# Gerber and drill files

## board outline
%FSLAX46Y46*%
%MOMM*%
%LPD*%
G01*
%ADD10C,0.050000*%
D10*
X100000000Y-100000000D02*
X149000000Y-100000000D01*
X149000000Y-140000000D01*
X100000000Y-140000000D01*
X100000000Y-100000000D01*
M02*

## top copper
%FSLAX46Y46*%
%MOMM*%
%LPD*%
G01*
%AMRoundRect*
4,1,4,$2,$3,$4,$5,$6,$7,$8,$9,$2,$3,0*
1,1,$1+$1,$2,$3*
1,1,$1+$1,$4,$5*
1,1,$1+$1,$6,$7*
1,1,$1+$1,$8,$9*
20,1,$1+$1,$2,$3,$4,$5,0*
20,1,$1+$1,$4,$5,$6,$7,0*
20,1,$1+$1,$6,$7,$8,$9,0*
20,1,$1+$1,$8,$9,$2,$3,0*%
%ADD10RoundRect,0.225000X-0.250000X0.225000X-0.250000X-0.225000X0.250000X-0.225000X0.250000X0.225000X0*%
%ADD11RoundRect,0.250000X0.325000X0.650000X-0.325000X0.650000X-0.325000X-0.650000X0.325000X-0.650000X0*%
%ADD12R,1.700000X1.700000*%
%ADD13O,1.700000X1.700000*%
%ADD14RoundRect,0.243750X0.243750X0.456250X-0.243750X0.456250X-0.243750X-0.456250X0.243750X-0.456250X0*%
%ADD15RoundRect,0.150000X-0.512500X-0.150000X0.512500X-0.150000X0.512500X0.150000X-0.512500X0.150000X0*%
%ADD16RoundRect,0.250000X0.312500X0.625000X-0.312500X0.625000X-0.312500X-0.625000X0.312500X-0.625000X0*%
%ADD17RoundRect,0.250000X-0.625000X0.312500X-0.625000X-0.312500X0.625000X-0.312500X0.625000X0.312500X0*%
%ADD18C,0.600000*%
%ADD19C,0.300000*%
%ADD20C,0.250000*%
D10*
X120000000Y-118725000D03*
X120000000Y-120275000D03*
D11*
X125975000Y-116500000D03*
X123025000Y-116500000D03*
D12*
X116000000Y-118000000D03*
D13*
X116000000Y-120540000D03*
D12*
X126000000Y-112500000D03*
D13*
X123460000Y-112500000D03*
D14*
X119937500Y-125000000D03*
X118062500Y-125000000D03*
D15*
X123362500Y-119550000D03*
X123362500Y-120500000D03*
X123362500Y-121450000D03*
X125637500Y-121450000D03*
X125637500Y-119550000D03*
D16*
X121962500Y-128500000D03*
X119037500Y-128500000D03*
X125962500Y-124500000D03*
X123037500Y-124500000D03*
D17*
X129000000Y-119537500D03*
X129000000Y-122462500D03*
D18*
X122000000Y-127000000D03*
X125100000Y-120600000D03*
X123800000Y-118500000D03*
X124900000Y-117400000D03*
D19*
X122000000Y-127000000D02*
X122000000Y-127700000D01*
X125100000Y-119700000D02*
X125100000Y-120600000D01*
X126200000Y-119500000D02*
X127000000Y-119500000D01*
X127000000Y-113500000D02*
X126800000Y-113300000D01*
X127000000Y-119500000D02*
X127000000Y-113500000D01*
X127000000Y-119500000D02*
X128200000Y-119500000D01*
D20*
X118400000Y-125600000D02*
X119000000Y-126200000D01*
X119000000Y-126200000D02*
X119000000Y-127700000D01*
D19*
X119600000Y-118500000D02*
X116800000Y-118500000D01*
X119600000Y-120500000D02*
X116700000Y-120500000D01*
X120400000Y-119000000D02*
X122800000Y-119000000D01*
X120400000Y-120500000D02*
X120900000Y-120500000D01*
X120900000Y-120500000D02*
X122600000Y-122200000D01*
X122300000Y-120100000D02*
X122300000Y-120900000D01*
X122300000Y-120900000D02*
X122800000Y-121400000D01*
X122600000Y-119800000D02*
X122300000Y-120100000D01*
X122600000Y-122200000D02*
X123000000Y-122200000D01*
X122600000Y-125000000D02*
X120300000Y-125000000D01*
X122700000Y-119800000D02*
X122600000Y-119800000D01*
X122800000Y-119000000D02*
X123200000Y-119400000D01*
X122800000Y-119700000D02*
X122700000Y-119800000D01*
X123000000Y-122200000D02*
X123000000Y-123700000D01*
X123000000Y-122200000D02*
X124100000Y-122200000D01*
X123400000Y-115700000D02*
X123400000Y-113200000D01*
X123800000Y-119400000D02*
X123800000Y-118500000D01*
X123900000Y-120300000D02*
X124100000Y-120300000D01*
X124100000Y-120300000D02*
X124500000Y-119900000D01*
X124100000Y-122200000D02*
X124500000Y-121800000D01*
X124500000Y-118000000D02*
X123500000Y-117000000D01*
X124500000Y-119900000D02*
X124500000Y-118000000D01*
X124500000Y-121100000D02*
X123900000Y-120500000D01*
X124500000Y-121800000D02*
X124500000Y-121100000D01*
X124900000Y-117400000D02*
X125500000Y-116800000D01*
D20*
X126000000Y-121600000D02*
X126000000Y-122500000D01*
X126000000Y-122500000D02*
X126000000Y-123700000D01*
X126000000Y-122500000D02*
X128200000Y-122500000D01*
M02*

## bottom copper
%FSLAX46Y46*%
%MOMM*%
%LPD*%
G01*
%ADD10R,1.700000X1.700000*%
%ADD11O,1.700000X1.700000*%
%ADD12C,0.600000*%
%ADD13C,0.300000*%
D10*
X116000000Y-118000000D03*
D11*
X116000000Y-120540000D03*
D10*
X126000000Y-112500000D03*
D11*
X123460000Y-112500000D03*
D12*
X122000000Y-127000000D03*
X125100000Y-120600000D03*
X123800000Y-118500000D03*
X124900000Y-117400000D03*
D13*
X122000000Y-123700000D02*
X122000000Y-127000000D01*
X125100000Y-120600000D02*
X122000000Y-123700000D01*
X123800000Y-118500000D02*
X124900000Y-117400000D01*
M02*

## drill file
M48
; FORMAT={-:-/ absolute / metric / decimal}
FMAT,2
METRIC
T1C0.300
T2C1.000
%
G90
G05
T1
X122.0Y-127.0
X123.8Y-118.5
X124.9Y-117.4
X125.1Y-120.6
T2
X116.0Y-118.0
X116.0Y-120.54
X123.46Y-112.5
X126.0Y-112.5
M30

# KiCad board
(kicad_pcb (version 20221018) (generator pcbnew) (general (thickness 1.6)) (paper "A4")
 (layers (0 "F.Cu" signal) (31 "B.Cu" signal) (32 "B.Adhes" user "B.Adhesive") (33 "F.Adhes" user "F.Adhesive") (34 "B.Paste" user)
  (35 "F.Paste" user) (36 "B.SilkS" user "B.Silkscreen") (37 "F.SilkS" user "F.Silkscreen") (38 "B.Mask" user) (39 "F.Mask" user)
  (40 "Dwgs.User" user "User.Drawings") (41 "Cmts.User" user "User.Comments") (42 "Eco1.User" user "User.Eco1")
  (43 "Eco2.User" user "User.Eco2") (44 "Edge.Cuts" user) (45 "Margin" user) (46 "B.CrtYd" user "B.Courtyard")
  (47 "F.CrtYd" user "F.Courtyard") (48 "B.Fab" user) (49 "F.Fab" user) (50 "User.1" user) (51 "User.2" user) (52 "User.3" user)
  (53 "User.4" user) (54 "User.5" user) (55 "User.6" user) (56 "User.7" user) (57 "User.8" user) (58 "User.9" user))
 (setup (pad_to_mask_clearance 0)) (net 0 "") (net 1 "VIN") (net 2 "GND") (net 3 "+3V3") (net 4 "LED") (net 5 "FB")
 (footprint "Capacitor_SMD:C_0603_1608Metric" (layer "F.Cu") (at 120 119.5 -90)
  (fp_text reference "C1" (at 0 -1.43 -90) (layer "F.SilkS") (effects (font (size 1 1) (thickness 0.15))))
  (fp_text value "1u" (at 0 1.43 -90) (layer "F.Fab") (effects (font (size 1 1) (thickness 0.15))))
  (pad "1" smd roundrect (at -0.775 0 270) (size 0.9 0.95) (layers "F.Cu" "F.Paste" "F.Mask") (roundrect_rratio 0.25) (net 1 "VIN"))
  (pad "2" smd roundrect (at 0.775 0 270) (size 0.9 0.95) (layers "F.Cu" "F.Paste" "F.Mask") (roundrect_rratio 0.25) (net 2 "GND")))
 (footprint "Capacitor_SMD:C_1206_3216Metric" (layer "F.Cu") (at 124.5 116.5 180)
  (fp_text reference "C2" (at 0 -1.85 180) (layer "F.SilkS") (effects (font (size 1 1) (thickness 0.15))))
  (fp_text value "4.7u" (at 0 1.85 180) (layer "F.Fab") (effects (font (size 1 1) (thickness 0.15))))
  (pad "1" smd roundrect (at -1.475 0 180) (size 1.15 1.8) (layers "F.Cu" "F.Paste" "F.Mask") (roundrect_rratio 0.217391) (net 1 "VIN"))
  (pad "2" smd roundrect (at 1.475 0 180) (size 1.15 1.8) (layers "F.Cu" "F.Paste" "F.Mask") (roundrect_rratio 0.217391) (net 2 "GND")))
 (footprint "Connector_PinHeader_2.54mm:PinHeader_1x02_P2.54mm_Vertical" (layer "F.Cu") (at 116 118)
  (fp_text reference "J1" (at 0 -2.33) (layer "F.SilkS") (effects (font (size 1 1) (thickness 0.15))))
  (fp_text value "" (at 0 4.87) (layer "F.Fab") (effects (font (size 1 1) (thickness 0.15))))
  (pad "1" thru_hole rect (at 0 0) (size 1.7 1.7) (drill 1) (layers "*.Cu" "*.Mask") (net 1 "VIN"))
  (pad "2" thru_hole oval (at 0 2.54) (size 1.7 1.7) (drill 1) (layers "*.Cu" "*.Mask") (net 2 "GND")))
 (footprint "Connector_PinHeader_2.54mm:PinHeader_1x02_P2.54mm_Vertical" (layer "F.Cu") (at 126 112.5 -90)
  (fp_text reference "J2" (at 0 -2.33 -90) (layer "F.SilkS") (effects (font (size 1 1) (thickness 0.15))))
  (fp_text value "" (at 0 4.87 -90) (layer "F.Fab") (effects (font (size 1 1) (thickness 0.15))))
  (pad "1" thru_hole rect (at 0 0 270) (size 1.7 1.7) (drill 1) (layers "*.Cu" "*.Mask") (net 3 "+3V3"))
  (pad "2" thru_hole oval (at 0 2.54 270) (size 1.7 1.7) (drill 1) (layers "*.Cu" "*.Mask") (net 2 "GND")))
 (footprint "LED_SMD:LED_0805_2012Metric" (layer "F.Cu") (at 119 125 180)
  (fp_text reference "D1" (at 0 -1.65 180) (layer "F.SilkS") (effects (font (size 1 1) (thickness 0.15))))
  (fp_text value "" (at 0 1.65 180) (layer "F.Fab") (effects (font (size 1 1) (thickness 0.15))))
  (pad "1" smd roundrect (at -0.9375 0 180) (size 0.975 1.4) (layers "F.Cu" "F.Paste" "F.Mask") (roundrect_rratio 0.25) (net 2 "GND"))
  (pad "2" smd roundrect (at 0.9375 0 180) (size 0.975 1.4) (layers "F.Cu" "F.Paste" "F.Mask") (roundrect_rratio 0.25) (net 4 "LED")))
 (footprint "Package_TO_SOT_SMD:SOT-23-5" (layer "F.Cu") (at 124.5 120.5)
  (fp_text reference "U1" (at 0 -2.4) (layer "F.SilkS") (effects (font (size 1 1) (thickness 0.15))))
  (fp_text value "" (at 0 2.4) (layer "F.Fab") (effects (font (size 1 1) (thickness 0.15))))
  (pad "1" smd roundrect (at -1.1375 -0.95) (size 1.325 0.6) (layers "F.Cu" "F.Paste" "F.Mask") (roundrect_rratio 0.25) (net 1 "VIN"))
  (pad "2" smd roundrect (at -1.1375 0) (size 1.325 0.6) (layers "F.Cu" "F.Paste" "F.Mask") (roundrect_rratio 0.25) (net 2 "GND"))
  (pad "3" smd roundrect (at -1.1375 0.95) (size 1.325 0.6) (layers "F.Cu" "F.Paste" "F.Mask") (roundrect_rratio 0.25) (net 1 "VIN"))
  (pad "4" smd roundrect (at 1.1375 0.95) (size 1.325 0.6) (layers "F.Cu" "F.Paste" "F.Mask") (roundrect_rratio 0.25) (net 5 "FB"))
  (pad "5" smd roundrect (at 1.1375 -0.95) (size 1.325 0.6) (layers "F.Cu" "F.Paste" "F.Mask") (roundrect_rratio 0.25) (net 3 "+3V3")))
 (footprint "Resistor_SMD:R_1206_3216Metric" (layer "F.Cu") (at 120.5 128.5 180)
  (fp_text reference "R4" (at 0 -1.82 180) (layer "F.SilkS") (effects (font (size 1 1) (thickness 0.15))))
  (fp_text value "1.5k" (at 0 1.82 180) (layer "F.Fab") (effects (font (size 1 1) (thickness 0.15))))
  (pad "1" smd roundrect (at -1.4625 0 180) (size 1.125 1.75) (layers "F.Cu" "F.Paste" "F.Mask") (roundrect_rratio 0.222222) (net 3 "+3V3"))
  (pad "2" smd roundrect (at 1.4625 0 180) (size 1.125 1.75) (layers "F.Cu" "F.Paste" "F.Mask") (roundrect_rratio 0.222222) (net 4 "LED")))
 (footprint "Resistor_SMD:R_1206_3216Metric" (layer "F.Cu") (at 124.5 124.5 180)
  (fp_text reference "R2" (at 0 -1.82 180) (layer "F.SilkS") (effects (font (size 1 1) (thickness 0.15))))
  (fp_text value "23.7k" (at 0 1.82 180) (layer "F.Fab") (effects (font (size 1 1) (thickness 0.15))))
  (pad "1" smd roundrect (at -1.4625 0 180) (size 1.125 1.75) (layers "F.Cu" "F.Paste" "F.Mask") (roundrect_rratio 0.222222) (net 5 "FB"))
  (pad "2" smd roundrect (at 1.4625 0 180) (size 1.125 1.75) (layers "F.Cu" "F.Paste" "F.Mask") (roundrect_rratio 0.222222) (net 2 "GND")))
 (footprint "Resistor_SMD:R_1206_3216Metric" (layer "F.Cu") (at 129 121 -90)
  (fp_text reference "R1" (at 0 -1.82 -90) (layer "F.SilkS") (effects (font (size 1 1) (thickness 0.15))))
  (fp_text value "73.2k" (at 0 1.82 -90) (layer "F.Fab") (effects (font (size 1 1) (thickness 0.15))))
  (pad "1" smd roundrect (at -1.4625 0 270) (size 1.125 1.75) (layers "F.Cu" "F.Paste" "F.Mask") (roundrect_rratio 0.222222) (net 3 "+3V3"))
  (pad "2" smd roundrect (at 1.4625 0 270) (size 1.125 1.75) (layers "F.Cu" "F.Paste" "F.Mask") (roundrect_rratio 0.222222) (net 5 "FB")))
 (gr_rect (start 100 100) (end 149 140) (stroke (width 0.05) (type default)) (fill none) (layer "Edge.Cuts"))
 (segment (start 122 127) (end 122 127.7) (width 0.3) (layer "F.Cu") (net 3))
 (segment (start 125.1 119.7) (end 125.1 120.6) (width 0.3) (layer "F.Cu") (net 3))
 (segment (start 126.2 119.5) (end 127 119.5) (width 0.3) (layer "F.Cu") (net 3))
 (segment (start 127 113.5) (end 126.8 113.3) (width 0.3) (layer "F.Cu") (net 3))
 (segment (start 127 119.5) (end 127 113.5) (width 0.3) (layer "F.Cu") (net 3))
 (segment (start 127 119.5) (end 128.2 119.5) (width 0.3) (layer "F.Cu") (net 3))
 (via (at 122 127) (size 0.6) (drill 0.3) (layers "F.Cu" "B.Cu") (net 3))
 (via (at 125.1 120.6) (size 0.6) (drill 0.3) (layers "F.Cu" "B.Cu") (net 3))
 (segment (start 118.4 125.6) (end 119 126.2) (width 0.25) (layer "F.Cu") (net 4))
 (segment (start 119 126.2) (end 119 127.7) (width 0.25) (layer "F.Cu") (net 4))
 (segment (start 119.6 118.5) (end 116.8 118.5) (width 0.3) (layer "F.Cu") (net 1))
 (segment (start 119.6 120.5) (end 116.7 120.5) (width 0.3) (layer "F.Cu") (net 2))
 (segment (start 120.4 119) (end 122.8 119) (width 0.3) (layer "F.Cu") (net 1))
 (segment (start 120.4 120.5) (end 120.9 120.5) (width 0.3) (layer "F.Cu") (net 2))
 (segment (start 120.9 120.5) (end 122.6 122.2) (width 0.3) (layer "F.Cu") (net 2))
 (segment (start 122 123.7) (end 122 127) (width 0.3) (layer "B.Cu") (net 3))
 (segment (start 122.3 120.1) (end 122.3 120.9) (width 0.3) (layer "F.Cu") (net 1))
 (segment (start 122.3 120.9) (end 122.8 121.4) (width 0.3) (layer "F.Cu") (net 1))
 (segment (start 122.6 119.8) (end 122.3 120.1) (width 0.3) (layer "F.Cu") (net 1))
 (segment (start 122.6 122.2) (end 123 122.2) (width 0.3) (layer "F.Cu") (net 2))
 (segment (start 122.6 125) (end 120.3 125) (width 0.3) (layer "F.Cu") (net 2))
 (segment (start 122.7 119.8) (end 122.6 119.8) (width 0.3) (layer "F.Cu") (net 1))
 (segment (start 122.8 119) (end 123.2 119.4) (width 0.3) (layer "F.Cu") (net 1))
 (segment (start 122.8 119.7) (end 122.7 119.8) (width 0.3) (layer "F.Cu") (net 1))
 (segment (start 123 122.2) (end 123 123.7) (width 0.3) (layer "F.Cu") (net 2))
 (segment (start 123 122.2) (end 124.1 122.2) (width 0.3) (layer "F.Cu") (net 2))
 (segment (start 123.4 115.7) (end 123.4 113.2) (width 0.3) (layer "F.Cu") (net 2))
 (segment (start 123.8 119.4) (end 123.8 118.5) (width 0.3) (layer "F.Cu") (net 1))
 (segment (start 123.9 120.3) (end 124.1 120.3) (width 0.3) (layer "F.Cu") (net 2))
 (segment (start 124.1 120.3) (end 124.5 119.9) (width 0.3) (layer "F.Cu") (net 2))
 (segment (start 124.1 122.2) (end 124.5 121.8) (width 0.3) (layer "F.Cu") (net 2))
 (segment (start 124.5 118) (end 123.5 117) (width 0.3) (layer "F.Cu") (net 2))
 (segment (start 124.5 119.9) (end 124.5 118) (width 0.3) (layer "F.Cu") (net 2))
 (segment (start 124.5 121.1) (end 123.9 120.5) (width 0.3) (layer "F.Cu") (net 2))
 (segment (start 124.5 121.8) (end 124.5 121.1) (width 0.3) (layer "F.Cu") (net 2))
 (segment (start 124.9 117.4) (end 125.5 116.8) (width 0.3) (layer "F.Cu") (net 1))
 (segment (start 125.1 120.6) (end 122 123.7) (width 0.3) (layer "B.Cu") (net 3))
 (segment (start 126 121.6) (end 126 122.5) (width 0.25) (layer "F.Cu") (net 5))
 (segment (start 126 122.5) (end 126 123.7) (width 0.25) (layer "F.Cu") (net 5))
 (segment (start 126 122.5) (end 128.2 122.5) (width 0.25) (layer "F.Cu") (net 5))
 (via (at 123.8 118.5) (size 0.6) (drill 0.3) (layers "F.Cu" "B.Cu") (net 1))
 (via (at 124.9 117.4) (size 0.6) (drill 0.3) (layers "F.Cu" "B.Cu") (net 1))
 (segment (start 123.8 118.5) (end 124.9 117.4) (width 0.3) (layer "B.Cu") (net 1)))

